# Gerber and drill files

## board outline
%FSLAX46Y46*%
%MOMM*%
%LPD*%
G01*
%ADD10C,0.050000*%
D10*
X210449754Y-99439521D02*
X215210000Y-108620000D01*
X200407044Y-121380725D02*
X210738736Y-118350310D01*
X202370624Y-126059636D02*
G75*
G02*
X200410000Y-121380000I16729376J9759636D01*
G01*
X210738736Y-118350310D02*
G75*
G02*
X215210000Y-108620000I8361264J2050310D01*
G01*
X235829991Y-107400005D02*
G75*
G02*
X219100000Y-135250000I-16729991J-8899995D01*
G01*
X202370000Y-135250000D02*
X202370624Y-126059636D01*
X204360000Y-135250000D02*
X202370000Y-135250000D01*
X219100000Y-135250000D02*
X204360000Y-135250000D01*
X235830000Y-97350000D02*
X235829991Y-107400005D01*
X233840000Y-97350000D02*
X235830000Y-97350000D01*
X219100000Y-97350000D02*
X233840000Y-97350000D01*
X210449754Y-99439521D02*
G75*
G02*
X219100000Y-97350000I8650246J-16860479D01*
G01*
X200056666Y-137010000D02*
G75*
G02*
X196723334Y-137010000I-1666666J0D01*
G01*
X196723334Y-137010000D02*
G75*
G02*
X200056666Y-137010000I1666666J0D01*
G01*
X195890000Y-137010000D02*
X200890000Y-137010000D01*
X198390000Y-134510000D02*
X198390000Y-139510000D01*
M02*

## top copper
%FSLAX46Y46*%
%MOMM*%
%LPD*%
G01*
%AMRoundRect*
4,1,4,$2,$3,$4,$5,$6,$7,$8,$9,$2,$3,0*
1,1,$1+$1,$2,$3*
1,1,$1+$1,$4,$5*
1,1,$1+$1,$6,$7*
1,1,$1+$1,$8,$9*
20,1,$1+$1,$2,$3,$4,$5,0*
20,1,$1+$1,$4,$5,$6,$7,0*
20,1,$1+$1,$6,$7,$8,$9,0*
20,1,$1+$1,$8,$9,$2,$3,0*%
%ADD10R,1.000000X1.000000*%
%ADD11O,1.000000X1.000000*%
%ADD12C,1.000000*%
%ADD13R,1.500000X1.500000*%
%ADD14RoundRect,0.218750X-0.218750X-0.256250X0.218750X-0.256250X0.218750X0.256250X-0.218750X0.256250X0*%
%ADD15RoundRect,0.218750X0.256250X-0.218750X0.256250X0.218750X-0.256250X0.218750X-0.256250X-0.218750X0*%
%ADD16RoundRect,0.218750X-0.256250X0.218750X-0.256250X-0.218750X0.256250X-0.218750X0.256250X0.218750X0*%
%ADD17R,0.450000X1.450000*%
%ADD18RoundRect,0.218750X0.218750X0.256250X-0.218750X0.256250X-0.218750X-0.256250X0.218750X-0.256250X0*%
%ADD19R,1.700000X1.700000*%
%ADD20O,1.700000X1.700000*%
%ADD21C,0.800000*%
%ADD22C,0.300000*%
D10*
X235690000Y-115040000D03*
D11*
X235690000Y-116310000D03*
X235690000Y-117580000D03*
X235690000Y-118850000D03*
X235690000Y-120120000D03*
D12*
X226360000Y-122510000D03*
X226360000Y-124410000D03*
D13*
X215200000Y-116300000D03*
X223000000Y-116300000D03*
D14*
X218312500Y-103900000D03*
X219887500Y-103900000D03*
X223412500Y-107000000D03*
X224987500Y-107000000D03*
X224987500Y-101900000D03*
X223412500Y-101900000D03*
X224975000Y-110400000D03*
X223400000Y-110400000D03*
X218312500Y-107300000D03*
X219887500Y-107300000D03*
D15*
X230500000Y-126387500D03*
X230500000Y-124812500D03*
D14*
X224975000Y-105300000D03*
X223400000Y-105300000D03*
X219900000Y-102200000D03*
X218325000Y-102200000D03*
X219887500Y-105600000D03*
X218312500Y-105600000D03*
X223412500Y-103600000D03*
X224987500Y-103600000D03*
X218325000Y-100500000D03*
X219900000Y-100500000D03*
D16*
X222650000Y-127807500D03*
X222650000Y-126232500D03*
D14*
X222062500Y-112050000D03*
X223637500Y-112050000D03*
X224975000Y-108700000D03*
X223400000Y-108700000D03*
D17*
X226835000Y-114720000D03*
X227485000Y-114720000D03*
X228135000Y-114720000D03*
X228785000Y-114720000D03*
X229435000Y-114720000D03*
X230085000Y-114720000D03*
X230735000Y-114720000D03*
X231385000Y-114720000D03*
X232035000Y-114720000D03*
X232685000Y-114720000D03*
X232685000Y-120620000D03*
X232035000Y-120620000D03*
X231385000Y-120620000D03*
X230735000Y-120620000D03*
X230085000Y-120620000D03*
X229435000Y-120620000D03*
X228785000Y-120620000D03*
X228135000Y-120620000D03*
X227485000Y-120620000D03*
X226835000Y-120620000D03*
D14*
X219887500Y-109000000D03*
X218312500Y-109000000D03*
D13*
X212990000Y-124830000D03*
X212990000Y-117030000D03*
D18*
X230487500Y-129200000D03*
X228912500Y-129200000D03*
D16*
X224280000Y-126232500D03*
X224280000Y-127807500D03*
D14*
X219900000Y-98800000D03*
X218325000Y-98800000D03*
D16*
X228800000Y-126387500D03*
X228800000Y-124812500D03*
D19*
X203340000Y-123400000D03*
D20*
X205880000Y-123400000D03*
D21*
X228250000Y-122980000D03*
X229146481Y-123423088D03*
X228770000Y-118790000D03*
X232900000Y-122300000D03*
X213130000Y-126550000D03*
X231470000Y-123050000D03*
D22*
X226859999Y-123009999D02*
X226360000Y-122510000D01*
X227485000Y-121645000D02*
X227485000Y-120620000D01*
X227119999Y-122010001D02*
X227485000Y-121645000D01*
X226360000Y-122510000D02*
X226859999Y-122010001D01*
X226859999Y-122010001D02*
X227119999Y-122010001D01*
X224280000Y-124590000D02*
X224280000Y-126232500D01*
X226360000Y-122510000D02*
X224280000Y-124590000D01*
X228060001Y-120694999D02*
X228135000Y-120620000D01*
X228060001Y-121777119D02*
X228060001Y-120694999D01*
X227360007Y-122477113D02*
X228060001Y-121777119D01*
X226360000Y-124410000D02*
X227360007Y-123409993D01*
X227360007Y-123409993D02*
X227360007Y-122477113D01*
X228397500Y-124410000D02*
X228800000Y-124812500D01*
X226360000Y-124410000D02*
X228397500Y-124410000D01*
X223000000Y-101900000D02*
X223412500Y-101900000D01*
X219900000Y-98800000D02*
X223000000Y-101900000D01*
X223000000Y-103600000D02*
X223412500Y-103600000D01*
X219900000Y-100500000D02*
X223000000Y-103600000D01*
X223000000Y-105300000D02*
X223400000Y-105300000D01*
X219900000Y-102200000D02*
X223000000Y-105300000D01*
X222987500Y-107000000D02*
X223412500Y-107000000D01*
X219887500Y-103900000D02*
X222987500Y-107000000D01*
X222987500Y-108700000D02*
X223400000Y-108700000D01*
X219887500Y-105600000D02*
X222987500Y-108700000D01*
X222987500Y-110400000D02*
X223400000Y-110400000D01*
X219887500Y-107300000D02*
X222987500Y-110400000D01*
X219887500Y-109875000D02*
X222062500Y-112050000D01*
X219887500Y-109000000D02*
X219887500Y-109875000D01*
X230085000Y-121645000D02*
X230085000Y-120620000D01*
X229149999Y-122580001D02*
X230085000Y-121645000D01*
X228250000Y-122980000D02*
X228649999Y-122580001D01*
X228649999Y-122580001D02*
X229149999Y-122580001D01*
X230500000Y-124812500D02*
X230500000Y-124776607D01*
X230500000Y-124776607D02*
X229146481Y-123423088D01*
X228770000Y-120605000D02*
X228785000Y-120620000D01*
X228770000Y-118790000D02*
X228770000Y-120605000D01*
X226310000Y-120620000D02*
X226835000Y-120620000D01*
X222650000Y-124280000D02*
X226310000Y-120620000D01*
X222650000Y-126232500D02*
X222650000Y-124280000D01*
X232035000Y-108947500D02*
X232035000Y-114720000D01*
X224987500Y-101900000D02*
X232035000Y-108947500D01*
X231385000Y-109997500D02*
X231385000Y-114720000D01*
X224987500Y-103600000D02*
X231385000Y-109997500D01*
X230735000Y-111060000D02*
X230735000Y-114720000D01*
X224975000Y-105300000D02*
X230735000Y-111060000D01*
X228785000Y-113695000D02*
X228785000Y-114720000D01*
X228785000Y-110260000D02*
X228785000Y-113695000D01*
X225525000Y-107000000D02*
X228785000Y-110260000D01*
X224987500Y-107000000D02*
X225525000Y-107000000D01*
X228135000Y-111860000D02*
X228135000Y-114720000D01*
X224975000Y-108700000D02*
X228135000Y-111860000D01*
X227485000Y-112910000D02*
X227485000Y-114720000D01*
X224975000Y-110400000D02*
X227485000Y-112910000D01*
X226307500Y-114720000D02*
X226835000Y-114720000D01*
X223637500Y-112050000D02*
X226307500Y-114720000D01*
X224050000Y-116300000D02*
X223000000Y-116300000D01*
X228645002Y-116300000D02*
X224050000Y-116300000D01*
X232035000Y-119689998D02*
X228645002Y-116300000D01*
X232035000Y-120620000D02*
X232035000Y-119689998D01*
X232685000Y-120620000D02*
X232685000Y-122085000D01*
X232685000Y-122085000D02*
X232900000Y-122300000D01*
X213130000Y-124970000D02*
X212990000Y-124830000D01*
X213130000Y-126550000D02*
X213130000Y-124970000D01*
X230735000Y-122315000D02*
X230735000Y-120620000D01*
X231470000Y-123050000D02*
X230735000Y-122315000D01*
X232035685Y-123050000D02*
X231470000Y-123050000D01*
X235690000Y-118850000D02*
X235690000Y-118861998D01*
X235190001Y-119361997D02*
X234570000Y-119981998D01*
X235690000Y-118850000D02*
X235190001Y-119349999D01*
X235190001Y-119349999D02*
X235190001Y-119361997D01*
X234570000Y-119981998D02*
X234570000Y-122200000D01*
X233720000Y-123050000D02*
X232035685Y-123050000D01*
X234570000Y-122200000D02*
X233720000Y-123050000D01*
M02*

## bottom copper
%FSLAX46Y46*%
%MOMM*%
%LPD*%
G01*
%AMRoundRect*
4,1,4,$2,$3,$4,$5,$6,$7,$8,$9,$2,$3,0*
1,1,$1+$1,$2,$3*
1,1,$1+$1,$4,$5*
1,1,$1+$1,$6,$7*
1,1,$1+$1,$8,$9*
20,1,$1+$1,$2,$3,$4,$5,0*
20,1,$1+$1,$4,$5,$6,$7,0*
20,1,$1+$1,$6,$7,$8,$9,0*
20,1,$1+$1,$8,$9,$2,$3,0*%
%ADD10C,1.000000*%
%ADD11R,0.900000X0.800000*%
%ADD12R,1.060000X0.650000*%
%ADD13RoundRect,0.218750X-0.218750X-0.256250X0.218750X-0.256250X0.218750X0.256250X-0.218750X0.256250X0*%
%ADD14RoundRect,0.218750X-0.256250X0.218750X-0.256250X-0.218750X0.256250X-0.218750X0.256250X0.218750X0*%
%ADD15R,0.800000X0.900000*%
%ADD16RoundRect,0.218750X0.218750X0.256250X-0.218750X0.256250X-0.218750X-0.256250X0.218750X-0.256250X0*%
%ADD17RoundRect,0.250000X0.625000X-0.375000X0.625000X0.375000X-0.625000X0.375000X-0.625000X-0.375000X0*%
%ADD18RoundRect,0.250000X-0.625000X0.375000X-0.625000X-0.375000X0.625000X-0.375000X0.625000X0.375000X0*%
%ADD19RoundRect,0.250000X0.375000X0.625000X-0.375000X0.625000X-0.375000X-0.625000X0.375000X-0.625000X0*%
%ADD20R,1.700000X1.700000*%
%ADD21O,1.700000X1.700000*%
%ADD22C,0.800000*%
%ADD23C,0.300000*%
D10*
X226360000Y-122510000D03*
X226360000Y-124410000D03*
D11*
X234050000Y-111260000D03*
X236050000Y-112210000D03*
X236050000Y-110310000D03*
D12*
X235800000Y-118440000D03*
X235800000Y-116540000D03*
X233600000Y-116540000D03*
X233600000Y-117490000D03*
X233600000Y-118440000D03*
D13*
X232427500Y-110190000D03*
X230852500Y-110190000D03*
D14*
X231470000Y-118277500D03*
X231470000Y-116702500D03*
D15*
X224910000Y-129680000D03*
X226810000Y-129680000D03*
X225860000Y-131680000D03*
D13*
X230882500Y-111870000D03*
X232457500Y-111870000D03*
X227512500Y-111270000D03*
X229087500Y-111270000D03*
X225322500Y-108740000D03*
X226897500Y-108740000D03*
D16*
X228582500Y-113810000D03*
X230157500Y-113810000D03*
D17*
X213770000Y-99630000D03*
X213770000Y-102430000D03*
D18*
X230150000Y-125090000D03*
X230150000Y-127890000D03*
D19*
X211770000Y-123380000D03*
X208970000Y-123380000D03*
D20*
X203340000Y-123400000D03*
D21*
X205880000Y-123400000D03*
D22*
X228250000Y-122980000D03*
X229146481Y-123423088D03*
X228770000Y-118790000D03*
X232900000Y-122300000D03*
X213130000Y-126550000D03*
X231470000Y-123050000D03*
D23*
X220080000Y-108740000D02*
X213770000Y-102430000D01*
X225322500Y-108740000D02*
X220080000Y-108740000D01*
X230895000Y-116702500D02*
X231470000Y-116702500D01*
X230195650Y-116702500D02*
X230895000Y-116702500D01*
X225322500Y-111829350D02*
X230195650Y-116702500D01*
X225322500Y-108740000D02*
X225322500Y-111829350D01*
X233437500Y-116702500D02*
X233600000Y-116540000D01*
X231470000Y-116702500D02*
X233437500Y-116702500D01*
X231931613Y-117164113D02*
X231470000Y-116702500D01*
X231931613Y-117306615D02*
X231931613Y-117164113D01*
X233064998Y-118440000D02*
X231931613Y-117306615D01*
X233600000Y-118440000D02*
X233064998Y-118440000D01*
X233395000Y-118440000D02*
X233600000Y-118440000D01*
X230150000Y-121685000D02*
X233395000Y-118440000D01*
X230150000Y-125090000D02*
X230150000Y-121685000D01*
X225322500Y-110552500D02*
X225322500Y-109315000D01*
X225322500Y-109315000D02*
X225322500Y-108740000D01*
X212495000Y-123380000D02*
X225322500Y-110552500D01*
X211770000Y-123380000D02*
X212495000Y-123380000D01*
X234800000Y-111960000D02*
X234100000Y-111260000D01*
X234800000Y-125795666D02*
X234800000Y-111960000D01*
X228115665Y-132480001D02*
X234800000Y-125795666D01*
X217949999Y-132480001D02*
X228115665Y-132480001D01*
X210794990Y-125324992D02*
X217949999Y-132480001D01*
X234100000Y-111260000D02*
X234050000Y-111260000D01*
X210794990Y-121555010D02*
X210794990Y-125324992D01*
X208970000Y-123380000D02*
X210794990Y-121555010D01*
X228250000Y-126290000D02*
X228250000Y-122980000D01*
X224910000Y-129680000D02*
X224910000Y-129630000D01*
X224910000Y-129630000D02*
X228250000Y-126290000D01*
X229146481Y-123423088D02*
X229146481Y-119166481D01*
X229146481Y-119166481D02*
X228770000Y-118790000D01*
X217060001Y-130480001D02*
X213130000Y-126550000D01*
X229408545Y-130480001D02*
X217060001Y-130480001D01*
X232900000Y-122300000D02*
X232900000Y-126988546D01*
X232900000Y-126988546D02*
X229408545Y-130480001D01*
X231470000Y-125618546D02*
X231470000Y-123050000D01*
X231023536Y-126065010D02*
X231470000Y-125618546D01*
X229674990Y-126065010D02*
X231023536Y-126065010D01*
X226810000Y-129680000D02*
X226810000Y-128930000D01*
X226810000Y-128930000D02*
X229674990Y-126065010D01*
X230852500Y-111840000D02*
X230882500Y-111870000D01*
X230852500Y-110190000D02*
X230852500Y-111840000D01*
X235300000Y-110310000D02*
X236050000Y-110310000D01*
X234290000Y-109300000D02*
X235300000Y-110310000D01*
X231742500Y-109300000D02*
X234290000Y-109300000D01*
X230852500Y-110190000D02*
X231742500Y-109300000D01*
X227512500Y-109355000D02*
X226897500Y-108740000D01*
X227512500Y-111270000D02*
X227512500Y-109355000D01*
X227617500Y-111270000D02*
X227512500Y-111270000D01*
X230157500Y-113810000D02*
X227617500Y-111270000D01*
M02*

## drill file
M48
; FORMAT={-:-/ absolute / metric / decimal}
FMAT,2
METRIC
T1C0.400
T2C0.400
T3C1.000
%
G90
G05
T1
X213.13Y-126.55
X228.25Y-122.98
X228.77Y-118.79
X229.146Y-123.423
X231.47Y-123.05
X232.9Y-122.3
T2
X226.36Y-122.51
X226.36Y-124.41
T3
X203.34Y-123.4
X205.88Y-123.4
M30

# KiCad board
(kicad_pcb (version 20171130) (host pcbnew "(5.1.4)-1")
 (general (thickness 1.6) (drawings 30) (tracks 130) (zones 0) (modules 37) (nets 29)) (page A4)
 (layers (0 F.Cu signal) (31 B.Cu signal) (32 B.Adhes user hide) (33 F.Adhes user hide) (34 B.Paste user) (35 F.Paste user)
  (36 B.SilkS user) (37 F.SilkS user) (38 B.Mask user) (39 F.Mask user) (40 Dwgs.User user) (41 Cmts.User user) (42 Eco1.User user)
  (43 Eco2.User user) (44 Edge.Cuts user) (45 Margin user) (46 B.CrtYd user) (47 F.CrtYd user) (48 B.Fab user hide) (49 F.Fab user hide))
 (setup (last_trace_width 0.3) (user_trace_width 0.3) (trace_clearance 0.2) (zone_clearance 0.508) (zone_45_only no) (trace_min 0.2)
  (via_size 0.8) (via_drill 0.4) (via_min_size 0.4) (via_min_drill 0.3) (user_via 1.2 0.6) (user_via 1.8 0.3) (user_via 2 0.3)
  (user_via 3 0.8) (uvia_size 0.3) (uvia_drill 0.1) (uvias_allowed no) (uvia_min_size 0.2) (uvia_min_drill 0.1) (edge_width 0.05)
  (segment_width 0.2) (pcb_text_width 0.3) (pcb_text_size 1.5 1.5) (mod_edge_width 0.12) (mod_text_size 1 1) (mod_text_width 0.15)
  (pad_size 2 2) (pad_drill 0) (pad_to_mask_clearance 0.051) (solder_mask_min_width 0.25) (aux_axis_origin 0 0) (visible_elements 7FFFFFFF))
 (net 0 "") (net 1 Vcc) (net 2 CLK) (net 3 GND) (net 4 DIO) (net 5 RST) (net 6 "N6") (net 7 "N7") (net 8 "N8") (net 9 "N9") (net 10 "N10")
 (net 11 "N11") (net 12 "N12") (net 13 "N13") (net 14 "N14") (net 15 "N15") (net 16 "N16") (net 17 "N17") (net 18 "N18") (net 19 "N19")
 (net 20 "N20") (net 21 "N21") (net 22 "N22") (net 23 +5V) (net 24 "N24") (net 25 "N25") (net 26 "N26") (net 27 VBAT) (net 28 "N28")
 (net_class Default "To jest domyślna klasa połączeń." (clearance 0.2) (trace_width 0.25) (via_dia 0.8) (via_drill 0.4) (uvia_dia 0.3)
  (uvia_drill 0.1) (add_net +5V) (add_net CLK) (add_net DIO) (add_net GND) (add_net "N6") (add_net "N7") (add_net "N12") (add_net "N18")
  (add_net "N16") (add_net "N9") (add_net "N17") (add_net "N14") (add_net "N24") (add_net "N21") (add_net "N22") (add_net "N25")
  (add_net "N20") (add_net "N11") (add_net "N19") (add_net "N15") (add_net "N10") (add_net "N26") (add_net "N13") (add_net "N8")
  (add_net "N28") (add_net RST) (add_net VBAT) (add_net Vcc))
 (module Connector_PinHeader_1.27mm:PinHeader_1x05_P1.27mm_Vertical (layer F.Cu) (at 235.69 115.04)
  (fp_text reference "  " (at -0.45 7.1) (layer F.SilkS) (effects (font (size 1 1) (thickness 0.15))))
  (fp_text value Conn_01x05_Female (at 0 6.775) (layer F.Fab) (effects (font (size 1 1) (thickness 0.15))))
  (pad 1 smd rect (at 0 0) (size 1 1) (layers F.Cu F.Paste F.Mask) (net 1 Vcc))
  (pad 2 smd oval (at 0 1.27) (size 1 1) (layers F.Cu F.Paste F.Mask) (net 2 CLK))
  (pad 3 smd oval (at 0 2.54) (size 1 1) (layers F.Cu F.Paste F.Mask) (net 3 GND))
  (pad 4 smd oval (at 0 3.81) (size 1 1) (layers F.Cu F.Paste F.Mask) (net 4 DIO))
  (pad 5 smd oval (at 0 5.08) (size 1 1) (layers F.Cu F.Paste F.Mask) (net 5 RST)))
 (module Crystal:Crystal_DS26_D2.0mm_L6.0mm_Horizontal (layer F.Cu) (at 226.36 122.51 270)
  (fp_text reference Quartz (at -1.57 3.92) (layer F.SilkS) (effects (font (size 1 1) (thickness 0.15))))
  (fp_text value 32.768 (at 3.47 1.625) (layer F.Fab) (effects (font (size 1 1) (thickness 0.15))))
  (pad 1 thru_hole circle (at 0 0 270) (size 1 1) (drill 0.4) (layers *.Cu *.Mask) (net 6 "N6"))
  (pad 2 thru_hole circle (at 1.9 0 270) (size 1 1) (drill 0.4) (layers *.Cu *.Mask) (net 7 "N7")))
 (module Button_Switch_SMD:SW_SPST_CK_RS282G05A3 (layer F.Cu) (at 219.1 116.3 180)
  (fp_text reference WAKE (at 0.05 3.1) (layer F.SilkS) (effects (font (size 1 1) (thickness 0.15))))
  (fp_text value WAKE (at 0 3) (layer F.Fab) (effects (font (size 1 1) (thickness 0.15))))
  (pad 2 smd rect (at 3.9 0 180) (size 1.5 1.5) (layers F.Cu F.Paste F.Mask) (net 3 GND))
  (pad 1 smd rect (at -3.9 0 180) (size 1.5 1.5) (layers F.Cu F.Paste F.Mask) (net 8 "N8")))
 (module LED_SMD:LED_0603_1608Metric (layer F.Cu) (at 219.1 103.9)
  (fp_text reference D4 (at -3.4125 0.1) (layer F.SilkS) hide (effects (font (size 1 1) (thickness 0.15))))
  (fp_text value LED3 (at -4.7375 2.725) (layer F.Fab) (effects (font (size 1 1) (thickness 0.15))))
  (pad 1 smd roundrect (at -0.7875 0) (size 0.875 0.95) (layers F.Cu F.Paste F.Mask) (roundrect_rratio 0.25) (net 3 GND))
  (pad 2 smd roundrect (at 0.7875 0) (size 0.875 0.95) (layers F.Cu F.Paste F.Mask) (roundrect_rratio 0.25) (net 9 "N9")))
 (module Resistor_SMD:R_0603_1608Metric (layer F.Cu) (at 224.2 107)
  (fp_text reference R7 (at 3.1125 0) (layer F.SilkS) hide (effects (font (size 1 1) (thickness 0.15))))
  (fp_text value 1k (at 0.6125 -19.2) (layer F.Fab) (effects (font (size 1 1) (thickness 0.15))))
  (pad 1 smd roundrect (at -0.7875 0) (size 0.875 0.95) (layers F.Cu F.Paste F.Mask) (roundrect_rratio 0.25) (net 9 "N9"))
  (pad 2 smd roundrect (at 0.7875 0) (size 0.875 0.95) (layers F.Cu F.Paste F.Mask) (roundrect_rratio 0.25) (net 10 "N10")))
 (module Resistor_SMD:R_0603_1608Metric (layer F.Cu) (at 224.2 101.9)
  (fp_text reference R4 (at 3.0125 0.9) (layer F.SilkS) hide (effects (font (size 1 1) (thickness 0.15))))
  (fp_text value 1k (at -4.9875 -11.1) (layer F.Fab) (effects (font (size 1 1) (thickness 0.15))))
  (pad 2 smd roundrect (at 0.7875 0) (size 0.875 0.95) (layers F.Cu F.Paste F.Mask) (roundrect_rratio 0.25) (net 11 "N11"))
  (pad 1 smd roundrect (at -0.7875 0) (size 0.875 0.95) (layers F.Cu F.Paste F.Mask) (roundrect_rratio 0.25) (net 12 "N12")))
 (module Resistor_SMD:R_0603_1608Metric (layer F.Cu) (at 224.1875 110.4)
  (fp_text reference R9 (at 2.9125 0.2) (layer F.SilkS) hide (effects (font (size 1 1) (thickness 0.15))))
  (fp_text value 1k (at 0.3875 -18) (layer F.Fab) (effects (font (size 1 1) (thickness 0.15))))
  (pad 2 smd roundrect (at 0.7875 0) (size 0.875 0.95) (layers F.Cu F.Paste F.Mask) (roundrect_rratio 0.25) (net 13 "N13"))
  (pad 1 smd roundrect (at -0.7875 0) (size 0.875 0.95) (layers F.Cu F.Paste F.Mask) (roundrect_rratio 0.25) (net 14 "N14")))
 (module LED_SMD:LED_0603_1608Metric (layer F.Cu) (at 219.1 107.3)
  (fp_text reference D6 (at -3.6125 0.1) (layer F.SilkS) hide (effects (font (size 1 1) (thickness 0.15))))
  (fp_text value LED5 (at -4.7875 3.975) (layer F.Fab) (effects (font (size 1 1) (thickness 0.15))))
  (pad 1 smd roundrect (at -0.7875 0) (size 0.875 0.95) (layers F.Cu F.Paste F.Mask) (roundrect_rratio 0.25) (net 3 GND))
  (pad 2 smd roundrect (at 0.7875 0) (size 0.875 0.95) (layers F.Cu F.Paste F.Mask) (roundrect_rratio 0.25) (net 14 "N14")))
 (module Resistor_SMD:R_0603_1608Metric (layer F.Cu) (at 230.5 125.6 90)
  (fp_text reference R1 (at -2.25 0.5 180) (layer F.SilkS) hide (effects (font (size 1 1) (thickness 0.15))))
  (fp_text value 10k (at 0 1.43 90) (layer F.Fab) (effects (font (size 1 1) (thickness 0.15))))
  (pad 1 smd roundrect (at -0.7875 0 90) (size 0.875 0.95) (layers F.Cu F.Paste F.Mask) (roundrect_rratio 0.25) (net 1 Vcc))
  (pad 2 smd roundrect (at 0.7875 0 90) (size 0.875 0.95) (layers F.Cu F.Paste F.Mask) (roundrect_rratio 0.25) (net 5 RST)))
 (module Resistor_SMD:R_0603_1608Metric (layer F.Cu) (at 224.1875 105.3)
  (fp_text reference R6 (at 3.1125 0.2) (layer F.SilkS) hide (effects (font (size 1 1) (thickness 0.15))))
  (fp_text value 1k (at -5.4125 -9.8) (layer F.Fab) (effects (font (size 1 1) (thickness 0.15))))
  (pad 2 smd roundrect (at 0.7875 0) (size 0.875 0.95) (layers F.Cu F.Paste F.Mask) (roundrect_rratio 0.25) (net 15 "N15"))
  (pad 1 smd roundrect (at -0.7875 0) (size 0.875 0.95) (layers F.Cu F.Paste F.Mask) (roundrect_rratio 0.25) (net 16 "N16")))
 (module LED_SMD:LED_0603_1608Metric (layer F.Cu) (at 219.1125 102.2)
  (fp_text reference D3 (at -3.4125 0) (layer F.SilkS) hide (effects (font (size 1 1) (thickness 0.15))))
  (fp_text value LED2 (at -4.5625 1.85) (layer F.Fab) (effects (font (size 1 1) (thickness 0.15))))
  (pad 2 smd roundrect (at 0.7875 0) (size 0.875 0.95) (layers F.Cu F.Paste F.Mask) (roundrect_rratio 0.25) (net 16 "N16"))
  (pad 1 smd roundrect (at -0.7875 0) (size 0.875 0.95) (layers F.Cu F.Paste F.Mask) (roundrect_rratio 0.25) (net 3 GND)))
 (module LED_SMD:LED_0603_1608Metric (layer F.Cu) (at 219.1 105.6)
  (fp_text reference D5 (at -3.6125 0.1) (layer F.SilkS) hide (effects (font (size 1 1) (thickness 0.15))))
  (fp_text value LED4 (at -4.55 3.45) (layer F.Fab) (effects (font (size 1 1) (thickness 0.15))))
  (pad 2 smd roundrect (at 0.7875 0) (size 0.875 0.95) (layers F.Cu F.Paste F.Mask) (roundrect_rratio 0.25) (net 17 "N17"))
  (pad 1 smd roundrect (at -0.7875 0) (size 0.875 0.95) (layers F.Cu F.Paste F.Mask) (roundrect_rratio 0.25) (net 3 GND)))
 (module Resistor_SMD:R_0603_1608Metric (layer F.Cu) (at 224.2 103.6)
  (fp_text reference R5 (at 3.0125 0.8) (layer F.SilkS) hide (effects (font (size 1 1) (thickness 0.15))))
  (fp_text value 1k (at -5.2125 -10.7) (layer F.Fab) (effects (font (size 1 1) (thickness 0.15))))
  (pad 1 smd roundrect (at -0.7875 0) (size 0.875 0.95) (layers F.Cu F.Paste F.Mask) (roundrect_rratio 0.25) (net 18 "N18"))
  (pad 2 smd roundrect (at 0.7875 0) (size 0.875 0.95) (layers F.Cu F.Paste F.Mask) (roundrect_rratio 0.25) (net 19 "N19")))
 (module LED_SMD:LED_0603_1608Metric (layer F.Cu) (at 219.1125 100.5)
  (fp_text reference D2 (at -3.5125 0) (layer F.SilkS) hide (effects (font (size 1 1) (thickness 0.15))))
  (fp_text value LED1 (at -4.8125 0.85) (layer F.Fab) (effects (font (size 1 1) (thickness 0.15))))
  (pad 1 smd roundrect (at -0.7875 0) (size 0.875 0.95) (layers F.Cu F.Paste F.Mask) (roundrect_rratio 0.25) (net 3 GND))
  (pad 2 smd roundrect (at 0.7875 0) (size 0.875 0.95) (layers F.Cu F.Paste F.Mask) (roundrect_rratio 0.25) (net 18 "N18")))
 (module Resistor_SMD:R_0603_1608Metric (layer F.Cu) (at 222.65 127.02 270)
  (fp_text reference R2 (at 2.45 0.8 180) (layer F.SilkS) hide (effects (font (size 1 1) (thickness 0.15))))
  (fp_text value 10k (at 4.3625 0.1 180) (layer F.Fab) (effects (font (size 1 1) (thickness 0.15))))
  (pad 2 smd roundrect (at 0.7875 0 270) (size 0.875 0.95) (layers F.Cu F.Paste F.Mask) (roundrect_rratio 0.25) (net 3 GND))
  (pad 1 smd roundrect (at -0.7875 0 270) (size 0.875 0.95) (layers F.Cu F.Paste F.Mask) (roundrect_rratio 0.25) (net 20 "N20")))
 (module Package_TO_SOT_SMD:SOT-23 (layer B.Cu) (at 235.05 111.26 180)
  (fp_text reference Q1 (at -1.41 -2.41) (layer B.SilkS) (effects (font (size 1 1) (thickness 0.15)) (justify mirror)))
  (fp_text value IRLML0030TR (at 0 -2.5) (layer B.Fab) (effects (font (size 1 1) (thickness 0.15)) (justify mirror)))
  (pad 3 smd rect (at 1 0 180) (size 0.9 0.8) (layers B.Cu B.Paste B.Mask) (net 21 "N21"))
  (pad 2 smd rect (at -1 -0.95 180) (size 0.9 0.8) (layers B.Cu B.Paste B.Mask) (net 3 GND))
  (pad 1 smd rect (at -1 0.95 180) (size 0.9 0.8) (layers B.Cu B.Paste B.Mask) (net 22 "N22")))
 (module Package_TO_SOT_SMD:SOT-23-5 (layer B.Cu) (at 234.7 117.49)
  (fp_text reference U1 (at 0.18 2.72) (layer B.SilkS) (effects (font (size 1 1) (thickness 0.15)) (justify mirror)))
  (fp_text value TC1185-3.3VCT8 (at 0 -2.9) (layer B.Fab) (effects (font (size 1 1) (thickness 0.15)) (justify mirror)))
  (pad 5 smd rect (at 1.1 0.95) (size 1.06 0.65) (layers B.Cu B.Paste B.Mask) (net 1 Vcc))
  (pad 4 smd rect (at 1.1 -0.95) (size 1.06 0.65) (layers B.Cu B.Paste B.Mask))
  (pad 3 smd rect (at -1.1 -0.95) (size 1.06 0.65) (layers B.Cu B.Paste B.Mask) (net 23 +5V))
  (pad 2 smd rect (at -1.1 0) (size 1.06 0.65) (layers B.Cu B.Paste B.Mask) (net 3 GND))
  (pad 1 smd rect (at -1.1 0.95) (size 1.06 0.65) (layers B.Cu B.Paste B.Mask) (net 23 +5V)))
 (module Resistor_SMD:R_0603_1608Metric (layer F.Cu) (at 222.85 112.05)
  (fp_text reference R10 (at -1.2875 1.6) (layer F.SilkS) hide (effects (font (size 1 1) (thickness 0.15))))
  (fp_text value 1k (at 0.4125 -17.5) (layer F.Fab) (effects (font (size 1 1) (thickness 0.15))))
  (pad 1 smd roundrect (at -0.7875 0) (size 0.875 0.95) (layers F.Cu F.Paste F.Mask) (roundrect_rratio 0.25) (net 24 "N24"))
  (pad 2 smd roundrect (at 0.7875 0) (size 0.875 0.95) (layers F.Cu F.Paste F.Mask) (roundrect_rratio 0.25) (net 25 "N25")))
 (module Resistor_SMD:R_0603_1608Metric (layer F.Cu) (at 224.1875 108.7)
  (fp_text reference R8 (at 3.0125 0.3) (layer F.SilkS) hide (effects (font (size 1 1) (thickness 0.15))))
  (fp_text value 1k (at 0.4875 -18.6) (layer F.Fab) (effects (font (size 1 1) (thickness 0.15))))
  (pad 2 smd roundrect (at 0.7875 0) (size 0.875 0.95) (layers F.Cu F.Paste F.Mask) (roundrect_rratio 0.25) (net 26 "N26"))
  (pad 1 smd roundrect (at -0.7875 0) (size 0.875 0.95) (layers F.Cu F.Paste F.Mask) (roundrect_rratio 0.25) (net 17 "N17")))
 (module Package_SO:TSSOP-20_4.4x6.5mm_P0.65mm (layer F.Cu) (at 229.76 117.67 90)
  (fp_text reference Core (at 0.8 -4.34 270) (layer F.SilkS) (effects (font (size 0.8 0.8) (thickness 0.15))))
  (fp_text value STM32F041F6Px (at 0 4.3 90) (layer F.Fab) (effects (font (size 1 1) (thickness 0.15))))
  (pad 20 smd rect (at 2.95 -2.925 90) (size 1.45 0.45) (layers F.Cu F.Paste F.Mask) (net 25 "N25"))
  (pad 19 smd rect (at 2.95 -2.275 90) (size 1.45 0.45) (layers F.Cu F.Paste F.Mask) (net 13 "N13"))
  (pad 18 smd rect (at 2.95 -1.625 90) (size 1.45 0.45) (layers F.Cu F.Paste F.Mask) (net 26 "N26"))
  (pad 17 smd rect (at 2.95 -0.975 90) (size 1.45 0.45) (layers F.Cu F.Paste F.Mask) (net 10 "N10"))
  (pad 16 smd rect (at 2.95 -0.325 90) (size 1.45 0.45) (layers F.Cu F.Paste F.Mask) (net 1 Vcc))
  (pad 15 smd rect (at 2.95 0.325 90) (size 1.45 0.45) (layers F.Cu F.Paste F.Mask) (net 3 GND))
  (pad 14 smd rect (at 2.95 0.975 90) (size 1.45 0.45) (layers F.Cu F.Paste F.Mask) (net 15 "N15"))
  (pad 13 smd rect (at 2.95 1.625 90) (size 1.45 0.45) (layers F.Cu F.Paste F.Mask) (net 19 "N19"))
  (pad 12 smd rect (at 2.95 2.275 90) (size 1.45 0.45) (layers F.Cu F.Paste F.Mask) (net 11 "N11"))
  (pad 11 smd rect (at 2.95 2.925 90) (size 1.45 0.45) (layers F.Cu F.Paste F.Mask) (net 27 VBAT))
  (pad 10 smd rect (at -2.95 2.925 90) (size 1.45 0.45) (layers F.Cu F.Paste F.Mask) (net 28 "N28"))
  (pad 9 smd rect (at -2.95 2.275 90) (size 1.45 0.45) (layers F.Cu F.Paste F.Mask) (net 8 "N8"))
  (pad 8 smd rect (at -2.95 1.625 90) (size 1.45 0.45) (layers F.Cu F.Paste F.Mask))
  (pad 7 smd rect (at -2.95 0.975 90) (size 1.45 0.45) (layers F.Cu F.Paste F.Mask) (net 4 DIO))
  (pad 6 smd rect (at -2.95 0.325 90) (size 1.45 0.45) (layers F.Cu F.Paste F.Mask) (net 2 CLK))
  (pad 5 smd rect (at -2.95 -0.325 90) (size 1.45 0.45) (layers F.Cu F.Paste F.Mask) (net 1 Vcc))
  (pad 4 smd rect (at -2.95 -0.975 90) (size 1.45 0.45) (layers F.Cu F.Paste F.Mask) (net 5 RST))
  (pad 3 smd rect (at -2.95 -1.625 90) (size 1.45 0.45) (layers F.Cu F.Paste F.Mask) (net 7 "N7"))
  (pad 2 smd rect (at -2.95 -2.275 90) (size 1.45 0.45) (layers F.Cu F.Paste F.Mask) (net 6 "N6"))
  (pad 1 smd rect (at -2.95 -2.925 90) (size 1.45 0.45) (layers F.Cu F.Paste F.Mask) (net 20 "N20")))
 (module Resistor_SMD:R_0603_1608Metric (layer B.Cu) (at 231.64 110.19)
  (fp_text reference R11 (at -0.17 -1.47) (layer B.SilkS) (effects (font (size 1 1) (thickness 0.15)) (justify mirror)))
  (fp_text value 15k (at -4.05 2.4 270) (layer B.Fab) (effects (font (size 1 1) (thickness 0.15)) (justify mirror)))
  (pad 2 smd roundrect (at 0.7875 0) (size 0.875 0.95) (layers B.Cu B.Paste B.Mask) (roundrect_rratio 0.25) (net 3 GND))
  (pad 1 smd roundrect (at -0.7875 0) (size 0.875 0.95) (layers B.Cu B.Paste B.Mask) (roundrect_rratio 0.25) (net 22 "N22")))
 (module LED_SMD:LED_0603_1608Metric (layer F.Cu) (at 219.1 109)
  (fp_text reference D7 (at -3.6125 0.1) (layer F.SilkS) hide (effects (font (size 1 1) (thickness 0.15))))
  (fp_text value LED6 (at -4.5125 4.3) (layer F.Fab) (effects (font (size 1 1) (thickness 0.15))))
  (pad 2 smd roundrect (at 0.7875 0) (size 0.875 0.95) (layers F.Cu F.Paste F.Mask) (roundrect_rratio 0.25) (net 24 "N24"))
  (pad 1 smd roundrect (at -0.7875 0) (size 0.875 0.95) (layers F.Cu F.Paste F.Mask) (roundrect_rratio 0.25) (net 3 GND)))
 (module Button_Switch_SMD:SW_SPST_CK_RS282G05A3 (layer F.Cu) (at 212.99 120.93 90)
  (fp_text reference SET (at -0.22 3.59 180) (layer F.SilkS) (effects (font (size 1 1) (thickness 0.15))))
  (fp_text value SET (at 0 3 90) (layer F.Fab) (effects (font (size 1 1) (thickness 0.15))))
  (pad 1 smd rect (at -3.9 0 90) (size 1.5 1.5) (layers F.Cu F.Paste F.Mask) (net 28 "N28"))
  (pad 2 smd rect (at 3.9 0 90) (size 1.5 1.5) (layers F.Cu F.Paste F.Mask) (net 3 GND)))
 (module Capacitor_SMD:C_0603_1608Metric (layer B.Cu) (at 231.47 117.49 270)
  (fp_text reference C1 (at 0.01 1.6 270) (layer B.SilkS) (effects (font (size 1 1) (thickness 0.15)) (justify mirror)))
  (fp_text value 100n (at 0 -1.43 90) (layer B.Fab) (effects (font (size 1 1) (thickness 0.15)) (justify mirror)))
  (pad 2 smd roundrect (at 0.7875 0 270) (size 0.875 0.95) (layers B.Cu B.Paste B.Mask) (roundrect_rratio 0.25) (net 3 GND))
  (pad 1 smd roundrect (at -0.7875 0 270) (size 0.875 0.95) (layers B.Cu B.Paste B.Mask) (roundrect_rratio 0.25) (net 23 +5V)))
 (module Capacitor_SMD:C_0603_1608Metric (layer F.Cu) (at 229.7 129.2 180)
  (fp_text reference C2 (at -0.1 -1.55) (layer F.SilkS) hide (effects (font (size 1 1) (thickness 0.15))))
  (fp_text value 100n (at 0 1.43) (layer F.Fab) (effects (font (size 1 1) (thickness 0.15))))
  (pad 1 smd roundrect (at -0.7875 0 180) (size 0.875 0.95) (layers F.Cu F.Paste F.Mask) (roundrect_rratio 0.25) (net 1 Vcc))
  (pad 2 smd roundrect (at 0.7875 0 180) (size 0.875 0.95) (layers F.Cu F.Paste F.Mask) (roundrect_rratio 0.25) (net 3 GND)))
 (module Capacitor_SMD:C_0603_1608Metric (layer F.Cu) (at 224.28 127.02 270)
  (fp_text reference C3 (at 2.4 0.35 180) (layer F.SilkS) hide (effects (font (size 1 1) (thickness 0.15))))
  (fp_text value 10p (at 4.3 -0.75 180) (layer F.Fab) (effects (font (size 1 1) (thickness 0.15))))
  (pad 1 smd roundrect (at -0.7875 0 270) (size 0.875 0.95) (layers F.Cu F.Paste F.Mask) (roundrect_rratio 0.25) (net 6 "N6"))
  (pad 2 smd roundrect (at 0.7875 0 270) (size 0.875 0.95) (layers F.Cu F.Paste F.Mask) (roundrect_rratio 0.25) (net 3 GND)))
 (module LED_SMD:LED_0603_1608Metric (layer F.Cu) (at 219.1125 98.8)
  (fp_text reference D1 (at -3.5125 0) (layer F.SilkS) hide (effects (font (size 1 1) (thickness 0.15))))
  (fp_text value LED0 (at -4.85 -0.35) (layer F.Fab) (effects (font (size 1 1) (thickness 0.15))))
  (pad 2 smd roundrect (at 0.7875 0) (size 0.875 0.95) (layers F.Cu F.Paste F.Mask) (roundrect_rratio 0.25) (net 12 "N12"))
  (pad 1 smd roundrect (at -0.7875 0) (size 0.875 0.95) (layers F.Cu F.Paste F.Mask) (roundrect_rratio 0.25) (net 3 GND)))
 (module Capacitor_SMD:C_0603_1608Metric (layer F.Cu) (at 228.8 125.6 270)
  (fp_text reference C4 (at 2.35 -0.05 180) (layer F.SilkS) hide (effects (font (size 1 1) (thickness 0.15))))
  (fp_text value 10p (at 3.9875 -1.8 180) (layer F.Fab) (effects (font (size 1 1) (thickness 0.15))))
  (pad 2 smd roundrect (at 0.7875 0 270) (size 0.875 0.95) (layers F.Cu F.Paste F.Mask) (roundrect_rratio 0.25) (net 3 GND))
  (pad 1 smd roundrect (at -0.7875 0 270) (size 0.875 0.95) (layers F.Cu F.Paste F.Mask) (roundrect_rratio 0.25) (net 7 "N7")))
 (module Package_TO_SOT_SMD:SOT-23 (layer B.Cu) (at 225.86 130.68 270)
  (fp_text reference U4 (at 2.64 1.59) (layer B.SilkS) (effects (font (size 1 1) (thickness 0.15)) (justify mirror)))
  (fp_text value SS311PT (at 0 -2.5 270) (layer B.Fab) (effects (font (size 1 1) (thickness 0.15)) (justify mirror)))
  (pad 1 smd rect (at -1 0.95 270) (size 0.9 0.8) (layers B.Cu B.Paste B.Mask) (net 2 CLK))
  (pad 2 smd rect (at -1 -0.95 270) (size 0.9 0.8) (layers B.Cu B.Paste B.Mask) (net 4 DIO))
  (pad 3 smd rect (at 1 0 270) (size 0.9 0.8) (layers B.Cu B.Paste B.Mask) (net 3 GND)))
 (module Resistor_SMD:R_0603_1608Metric (layer B.Cu) (at 231.67 111.87)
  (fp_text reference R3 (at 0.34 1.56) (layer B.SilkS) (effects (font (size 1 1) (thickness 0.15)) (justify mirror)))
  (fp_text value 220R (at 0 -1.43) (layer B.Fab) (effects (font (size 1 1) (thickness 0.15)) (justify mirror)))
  (pad 1 smd roundrect (at -0.7875 0) (size 0.875 0.95) (layers B.Cu B.Paste B.Mask) (roundrect_rratio 0.25) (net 22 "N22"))
  (pad 2 smd roundrect (at 0.7875 0) (size 0.875 0.95) (layers B.Cu B.Paste B.Mask) (roundrect_rratio 0.25) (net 2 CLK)))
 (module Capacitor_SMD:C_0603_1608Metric (layer B.Cu) (at 228.3 111.27)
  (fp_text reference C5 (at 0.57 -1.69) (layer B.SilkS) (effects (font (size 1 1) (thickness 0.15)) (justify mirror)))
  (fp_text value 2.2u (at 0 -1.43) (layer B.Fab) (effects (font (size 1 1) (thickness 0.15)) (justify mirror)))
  (pad 1 smd roundrect (at -0.7875 0) (size 0.875 0.95) (layers B.Cu B.Paste B.Mask) (roundrect_rratio 0.25) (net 27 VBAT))
  (pad 2 smd roundrect (at 0.7875 0) (size 0.875 0.95) (layers B.Cu B.Paste B.Mask) (roundrect_rratio 0.25) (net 3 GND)))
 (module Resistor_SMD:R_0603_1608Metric (layer B.Cu) (at 226.11 108.74)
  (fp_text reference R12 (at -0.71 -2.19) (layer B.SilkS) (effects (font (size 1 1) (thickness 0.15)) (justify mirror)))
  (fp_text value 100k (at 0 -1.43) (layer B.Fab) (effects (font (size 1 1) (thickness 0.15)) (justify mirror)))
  (pad 1 smd roundrect (at -0.7875 0) (size 0.875 0.95) (layers B.Cu B.Paste B.Mask) (roundrect_rratio 0.25) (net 23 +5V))
  (pad 2 smd roundrect (at 0.7875 0) (size 0.875 0.95) (layers B.Cu B.Paste B.Mask) (roundrect_rratio 0.25) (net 27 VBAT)))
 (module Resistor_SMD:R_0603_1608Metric (layer B.Cu) (at 229.37 113.81 180)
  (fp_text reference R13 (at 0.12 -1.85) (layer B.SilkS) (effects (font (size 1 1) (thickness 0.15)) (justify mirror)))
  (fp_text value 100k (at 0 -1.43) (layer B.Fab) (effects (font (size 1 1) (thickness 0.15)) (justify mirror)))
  (pad 2 smd roundrect (at 0.7875 0 180) (size 0.875 0.95) (layers B.Cu B.Paste B.Mask) (roundrect_rratio 0.25) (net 3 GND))
  (pad 1 smd roundrect (at -0.7875 0 180) (size 0.875 0.95) (layers B.Cu B.Paste B.Mask) (roundrect_rratio 0.25) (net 27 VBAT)))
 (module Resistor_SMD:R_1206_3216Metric (layer B.Cu) (at 213.77 101.03 90)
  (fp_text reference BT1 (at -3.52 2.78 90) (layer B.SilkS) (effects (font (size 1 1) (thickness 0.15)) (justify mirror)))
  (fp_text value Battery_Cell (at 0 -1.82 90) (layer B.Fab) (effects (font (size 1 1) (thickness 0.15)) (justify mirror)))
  (pad 2 smd roundrect (at 1.4 0 90) (size 1.25 1.75) (layers B.Cu B.Paste B.Mask) (roundrect_rratio 0.2) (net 3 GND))
  (pad 1 smd roundrect (at -1.4 0 90) (size 1.25 1.75) (layers B.Cu B.Paste B.Mask) (roundrect_rratio 0.2) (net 23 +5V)))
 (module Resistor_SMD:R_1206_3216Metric (layer B.Cu) (at 230.15 126.49 270)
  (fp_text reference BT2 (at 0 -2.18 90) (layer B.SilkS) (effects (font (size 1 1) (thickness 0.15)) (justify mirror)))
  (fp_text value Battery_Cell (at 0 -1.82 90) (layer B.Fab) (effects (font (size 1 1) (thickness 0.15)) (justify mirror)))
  (pad 1 smd roundrect (at -1.4 0 270) (size 1.25 1.75) (layers B.Cu B.Paste B.Mask) (roundrect_rratio 0.2) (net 23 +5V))
  (pad 2 smd roundrect (at 1.4 0 270) (size 1.25 1.75) (layers B.Cu B.Paste B.Mask) (roundrect_rratio 0.2) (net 3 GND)))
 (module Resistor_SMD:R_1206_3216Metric (layer B.Cu) (at 210.37 123.38 180)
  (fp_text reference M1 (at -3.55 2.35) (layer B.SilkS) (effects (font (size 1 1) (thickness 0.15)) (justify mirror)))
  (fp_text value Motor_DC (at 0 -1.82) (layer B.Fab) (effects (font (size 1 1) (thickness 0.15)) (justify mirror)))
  (pad 1 smd roundrect (at -1.4 0 180) (size 1.25 1.75) (layers B.Cu B.Paste B.Mask) (roundrect_rratio 0.2) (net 23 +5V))
  (pad 2 smd roundrect (at 1.4 0 180) (size 1.25 1.75) (layers B.Cu B.Paste B.Mask) (roundrect_rratio 0.2) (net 21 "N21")))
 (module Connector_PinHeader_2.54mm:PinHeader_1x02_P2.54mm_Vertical (layer F.Cu) (at 203.34 123.4 90)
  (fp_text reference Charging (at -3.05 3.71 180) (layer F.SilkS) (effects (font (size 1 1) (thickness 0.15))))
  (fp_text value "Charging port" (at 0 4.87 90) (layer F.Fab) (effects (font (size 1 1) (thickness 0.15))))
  (pad 1 thru_hole rect (at 0 0 90) (size 1.7 1.7) (drill 1) (layers *.Cu *.Mask) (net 3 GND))
  (pad 2 thru_hole oval (at 0 2.54 90) (size 1.7 1.7) (drill 1) (layers *.Cu *.Mask) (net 23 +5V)))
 (gr_line (start 210.449754 99.439521) (end 215.21 108.62) (layer Edge.Cuts) (width 0.05))
 (gr_line (start 200.407044 121.380725) (end 210.738736 118.35031) (layer Edge.Cuts) (width 0.05))
 (gr_arc (start 219.1 116.3) (end 200.41 121.38) (angle -15.05274458) (layer Edge.Cuts) (width 0.05))
 (gr_arc (start 219.1 116.3) (end 215.21 108.62) (angle -76.91524935) (layer Edge.Cuts) (width 0.05))
 (gr_arc (start 219.1 116.3) (end 219.1 135.25) (angle -118.0120165) (layer Edge.Cuts) (width 0.05))
 (gr_line (start 202.37 135.25) (end 202.370624 126.059636) (layer Edge.Cuts) (width 0.05))
 (gr_line (start 204.36 135.25) (end 202.37 135.25) (layer Edge.Cuts) (width 0.05))
 (gr_line (start 219.1 135.25) (end 204.36 135.25) (layer Edge.Cuts) (width 0.05))
 (gr_line (start 235.83 97.35) (end 235.829991 107.400005) (layer Edge.Cuts) (width 0.05))
 (gr_line (start 233.84 97.35) (end 235.83 97.35) (layer Edge.Cuts) (width 0.05))
 (gr_line (start 219.1 97.35) (end 233.84 97.35) (layer Edge.Cuts) (width 0.05))
 (gr_arc (start 219.1 116.3) (end 219.1 97.35) (angle -27.16002962) (layer Edge.Cuts) (width 0.05))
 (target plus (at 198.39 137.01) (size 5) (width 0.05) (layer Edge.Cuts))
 (segment (start 220.08 108.74) (end 213.77 102.43) (width 0.3) (layer B.Cu) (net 23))
 (segment (start 225.3225 108.74) (end 220.08 108.74) (width 0.3) (layer B.Cu) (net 23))
 (segment (start 230.895 116.7025) (end 231.47 116.7025) (width 0.3) (layer B.Cu) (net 23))
 (segment (start 230.19565 116.7025) (end 230.895 116.7025) (width 0.3) (layer B.Cu) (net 23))
 (segment (start 225.3225 111.82935) (end 230.19565 116.7025) (width 0.3) (layer B.Cu) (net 23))
 (segment (start 225.3225 108.74) (end 225.3225 111.82935) (width 0.3) (layer B.Cu) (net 23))
 (segment (start 233.4375 116.7025) (end 233.6 116.54) (width 0.3) (layer B.Cu) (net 23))
 (segment (start 231.47 116.7025) (end 233.4375 116.7025) (width 0.3) (layer B.Cu) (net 23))
 (segment (start 231.931613 117.164113) (end 231.47 116.7025) (width 0.3) (layer B.Cu) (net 23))
 (segment (start 231.931613 117.306615) (end 231.931613 117.164113) (width 0.3) (layer B.Cu) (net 23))
 (segment (start 233.064998 118.44) (end 231.931613 117.306615) (width 0.3) (layer B.Cu) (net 23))
 (segment (start 233.6 118.44) (end 233.064998 118.44) (width 0.3) (layer B.Cu) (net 23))
 (segment (start 233.395 118.44) (end 233.6 118.44) (width 0.3) (layer B.Cu) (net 23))
 (segment (start 230.15 121.685) (end 233.395 118.44) (width 0.3) (layer B.Cu) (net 23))
 (segment (start 230.15 125.09) (end 230.15 121.685) (width 0.3) (layer B.Cu) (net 23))
 (segment (start 225.3225 110.5525) (end 225.3225 109.315) (width 0.3) (layer B.Cu) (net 23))
 (segment (start 225.3225 109.315) (end 225.3225 108.74) (width 0.3) (layer B.Cu) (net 23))
 (segment (start 212.495 123.38) (end 225.3225 110.5525) (width 0.3) (layer B.Cu) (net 23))
 (segment (start 211.77 123.38) (end 212.495 123.38) (width 0.3) (layer B.Cu) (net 23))
 (segment (start 226.859999 123.009999) (end 226.36 122.51) (width 0.3) (layer F.Cu) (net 6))
 (segment (start 227.485 121.645) (end 227.485 120.62) (width 0.3) (layer F.Cu) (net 6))
 (segment (start 227.119999 122.010001) (end 227.485 121.645) (width 0.3) (layer F.Cu) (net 6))
 (segment (start 226.36 122.51) (end 226.859999 122.010001) (width 0.3) (layer F.Cu) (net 6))
 (segment (start 226.859999 122.010001) (end 227.119999 122.010001) (width 0.3) (layer F.Cu) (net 6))
 (segment (start 224.28 124.59) (end 224.28 126.2325) (width 0.3) (layer F.Cu) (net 6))
 (segment (start 226.36 122.51) (end 224.28 124.59) (width 0.3) (layer F.Cu) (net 6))
 (segment (start 228.060001 120.694999) (end 228.135 120.62) (width 0.3) (layer F.Cu) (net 7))
 (segment (start 228.060001 121.777119) (end 228.060001 120.694999) (width 0.3) (layer F.Cu) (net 7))
 (segment (start 227.360007 122.477113) (end 228.060001 121.777119) (width 0.3) (layer F.Cu) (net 7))
 (segment (start 226.36 124.41) (end 227.360007 123.409993) (width 0.3) (layer F.Cu) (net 7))
 (segment (start 227.360007 123.409993) (end 227.360007 122.477113) (width 0.3) (layer F.Cu) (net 7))
 (segment (start 228.3975 124.41) (end 228.8 124.8125) (width 0.3) (layer F.Cu) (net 7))
 (segment (start 226.36 124.41) (end 228.3975 124.41) (width 0.3) (layer F.Cu) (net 7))
 (segment (start 223 101.9) (end 223.4125 101.9) (width 0.3) (layer F.Cu) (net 12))
 (segment (start 219.9 98.8) (end 223 101.9) (width 0.3) (layer F.Cu) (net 12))
 (segment (start 223 103.6) (end 223.4125 103.6) (width 0.3) (layer F.Cu) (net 18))
 (segment (start 219.9 100.5) (end 223 103.6) (width 0.3) (layer F.Cu) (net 18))
 (segment (start 223 105.3) (end 223.4 105.3) (width 0.3) (layer F.Cu) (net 16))
 (segment (start 219.9 102.2) (end 223 105.3) (width 0.3) (layer F.Cu) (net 16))
 (segment (start 222.9875 107) (end 223.4125 107) (width 0.3) (layer F.Cu) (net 9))
 (segment (start 219.8875 103.9) (end 222.9875 107) (width 0.3) (layer F.Cu) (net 9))
 (segment (start 222.9875 108.7) (end 223.4 108.7) (width 0.3) (layer F.Cu) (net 17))
 (segment (start 219.8875 105.6) (end 222.9875 108.7) (width 0.3) (layer F.Cu) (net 17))
 (segment (start 222.9875 110.4) (end 223.4 110.4) (width 0.3) (layer F.Cu) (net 14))
 (segment (start 219.8875 107.3) (end 222.9875 110.4) (width 0.3) (layer F.Cu) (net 14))
 (segment (start 219.8875 109.875) (end 222.0625 112.05) (width 0.3) (layer F.Cu) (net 24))
 (segment (start 219.8875 109) (end 219.8875 109.875) (width 0.3) (layer F.Cu) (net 24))
 (segment (start 234.8 111.96) (end 234.1 111.26) (width 0.3) (layer B.Cu) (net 21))
 (segment (start 234.8 125.795666) (end 234.8 111.96) (width 0.3) (layer B.Cu) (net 21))
 (segment (start 228.115665 132.480001) (end 234.8 125.795666) (width 0.3) (layer B.Cu) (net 21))
 (segment (start 217.949999 132.480001) (end 228.115665 132.480001) (width 0.3) (layer B.Cu) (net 21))
 (segment (start 210.79499 125.324992) (end 217.949999 132.480001) (width 0.3) (layer B.Cu) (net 21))
 (segment (start 234.1 111.26) (end 234.05 111.26) (width 0.3) (layer B.Cu) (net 21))
 (segment (start 210.79499 121.55501) (end 210.79499 125.324992) (width 0.3) (layer B.Cu) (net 21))
 (segment (start 208.97 123.38) (end 210.79499 121.55501) (width 0.3) (layer B.Cu) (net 21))
 (via (at 228.25 122.98) (size 0.8) (drill 0.4) (layers F.Cu B.Cu) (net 2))
 (segment (start 228.25 126.29) (end 228.25 122.98) (width 0.3) (layer B.Cu) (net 2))
 (segment (start 224.91 129.68) (end 224.91 129.63) (width 0.3) (layer B.Cu) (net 2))
 (segment (start 224.91 129.63) (end 228.25 126.29) (width 0.3) (layer B.Cu) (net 2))
 (segment (start 230.085 121.645) (end 230.085 120.62) (width 0.3) (layer F.Cu) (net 2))
 (segment (start 229.149999 122.580001) (end 230.085 121.645) (width 0.3) (layer F.Cu) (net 2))
 (segment (start 228.25 122.98) (end 228.649999 122.580001) (width 0.3) (layer F.Cu) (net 2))
 (segment (start 228.649999 122.580001) (end 229.149999 122.580001) (width 0.3) (layer F.Cu) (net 2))
 (via (at 229.146481 123.423088) (size 0.8) (drill 0.4) (layers F.Cu B.Cu) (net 5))
 (segment (start 230.5 124.8125) (end 230.5 124.776607) (width 0.3) (layer F.Cu) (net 5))
 (segment (start 230.5 124.776607) (end 229.146481 123.423088) (width 0.3) (layer F.Cu) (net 5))
 (via (at 228.77 118.79) (size 0.8) (drill 0.4) (layers F.Cu B.Cu) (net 5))
 (segment (start 229.146481 123.423088) (end 229.146481 119.166481) (width 0.3) (layer B.Cu) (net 5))
 (segment (start 229.146481 119.166481) (end 228.77 118.79) (width 0.3) (layer B.Cu) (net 5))
 (segment (start 228.77 120.605) (end 228.785 120.62) (width 0.3) (layer F.Cu) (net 5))
 (segment (start 228.77 118.79) (end 228.77 120.605) (width 0.3) (layer F.Cu) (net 5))
 (segment (start 226.31 120.62) (end 226.835 120.62) (width 0.3) (layer F.Cu) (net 20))
 (segment (start 222.65 124.28) (end 226.31 120.62) (width 0.3) (layer F.Cu) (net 20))
 (segment (start 222.65 126.2325) (end 222.65 124.28) (width 0.3) (layer F.Cu) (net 20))
 (segment (start 232.035 108.9475) (end 232.035 114.72) (width 0.3) (layer F.Cu) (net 11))
 (segment (start 224.9875 101.9) (end 232.035 108.9475) (width 0.3) (layer F.Cu) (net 11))
 (segment (start 231.385 109.9975) (end 231.385 114.72) (width 0.3) (layer F.Cu) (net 19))
 (segment (start 224.9875 103.6) (end 231.385 109.9975) (width 0.3) (layer F.Cu) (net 19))
 (segment (start 230.735 111.06) (end 230.735 114.72) (width 0.3) (layer F.Cu) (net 15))
 (segment (start 224.975 105.3) (end 230.735 111.06) (width 0.3) (layer F.Cu) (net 15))
 (segment (start 228.785 113.695) (end 228.785 114.72) (width 0.3) (layer F.Cu) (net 10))
 (segment (start 228.785 110.26) (end 228.785 113.695) (width 0.3) (layer F.Cu) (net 10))
 (segment (start 225.525 107) (end 228.785 110.26) (width 0.3) (layer F.Cu) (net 10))
 (segment (start 224.9875 107) (end 225.525 107) (width 0.3) (layer F.Cu) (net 10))
 (segment (start 228.135 111.86) (end 228.135 114.72) (width 0.3) (layer F.Cu) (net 26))
 (segment (start 224.975 108.7) (end 228.135 111.86) (width 0.3) (layer F.Cu) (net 26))
 (segment (start 227.485 112.91) (end 227.485 114.72) (width 0.3) (layer F.Cu) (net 13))
 (segment (start 224.975 110.4) (end 227.485 112.91) (width 0.3) (layer F.Cu) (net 13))
 (segment (start 226.3075 114.72) (end 226.835 114.72) (width 0.3) (layer F.Cu) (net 25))
 (segment (start 223.6375 112.05) (end 226.3075 114.72) (width 0.3) (layer F.Cu) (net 25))
 (segment (start 224.05 116.3) (end 223 116.3) (width 0.3) (layer F.Cu) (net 8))
 (segment (start 228.645002 116.3) (end 224.05 116.3) (width 0.3) (layer F.Cu) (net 8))
 (segment (start 232.035 119.689998) (end 228.645002 116.3) (width 0.3) (layer F.Cu) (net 8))
 (segment (start 232.035 120.62) (end 232.035 119.689998) (width 0.3) (layer F.Cu) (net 8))
 (via (at 232.9 122.3) (size 0.8) (drill 0.4) (layers F.Cu B.Cu) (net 28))
 (segment (start 232.685 120.62) (end 232.685 122.085) (width 0.3) (layer F.Cu) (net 28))
 (segment (start 232.685 122.085) (end 232.9 122.3) (width 0.3) (layer F.Cu) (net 28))
 (via (at 213.13 126.55) (size 0.8) (drill 0.4) (layers F.Cu B.Cu) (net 28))
 (segment (start 217.060001 130.480001) (end 213.13 126.55) (width 0.3) (layer B.Cu) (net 28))
 (segment (start 229.408545 130.480001) (end 217.060001 130.480001) (width 0.3) (layer B.Cu) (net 28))
 (segment (start 232.9 122.3) (end 232.9 126.988546) (width 0.3) (layer B.Cu) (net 28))
 (segment (start 232.9 126.988546) (end 229.408545 130.480001) (width 0.3) (layer B.Cu) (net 28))
 (segment (start 213.13 124.97) (end 212.99 124.83) (width 0.3) (layer F.Cu) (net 28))
 (segment (start 213.13 126.55) (end 213.13 124.97) (width 0.3) (layer F.Cu) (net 28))
 (segment (start 231.47 125.618546) (end 231.47 123.05) (width 0.3) (layer B.Cu) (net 4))
 (via (at 231.47 123.05) (size 0.8) (drill 0.4) (layers F.Cu B.Cu) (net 4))
 (segment (start 231.023536 126.06501) (end 231.47 125.618546) (width 0.3) (layer B.Cu) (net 4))
 (segment (start 229.67499 126.06501) (end 231.023536 126.06501) (width 0.3) (layer B.Cu) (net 4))
 (segment (start 226.81 129.68) (end 226.81 128.93) (width 0.3) (layer B.Cu) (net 4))
 (segment (start 226.81 128.93) (end 229.67499 126.06501) (width 0.3) (layer B.Cu) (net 4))
 (segment (start 230.735 122.315) (end 230.735 120.62) (width 0.3) (layer F.Cu) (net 4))
 (segment (start 231.47 123.05) (end 230.735 122.315) (width 0.3) (layer F.Cu) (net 4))
 (segment (start 232.035685 123.05) (end 231.47 123.05) (width 0.3) (layer F.Cu) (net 4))
 (segment (start 235.69 118.85) (end 235.69 118.861998) (width 0.3) (layer F.Cu) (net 4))
 (segment (start 235.190001 119.361997) (end 234.57 119.981998) (width 0.3) (layer F.Cu) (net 4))
 (segment (start 235.69 118.85) (end 235.190001 119.349999) (width 0.3) (layer F.Cu) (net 4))
 (segment (start 235.190001 119.349999) (end 235.190001 119.361997) (width 0.3) (layer F.Cu) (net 4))
 (segment (start 234.57 119.981998) (end 234.57 122.2) (width 0.3) (layer F.Cu) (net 4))
 (segment (start 233.72 123.05) (end 232.035685 123.05) (width 0.3) (layer F.Cu) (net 4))
 (segment (start 234.57 122.2) (end 233.72 123.05) (width 0.3) (layer F.Cu) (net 4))
 (segment (start 230.8525 111.84) (end 230.8825 111.87) (width 0.3) (layer B.Cu) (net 22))
 (segment (start 230.8525 110.19) (end 230.8525 111.84) (width 0.3) (layer B.Cu) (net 22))
 (segment (start 235.3 110.31) (end 236.05 110.31) (width 0.3) (layer B.Cu) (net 22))
 (segment (start 234.29 109.3) (end 235.3 110.31) (width 0.3) (layer B.Cu) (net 22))
 (segment (start 231.7425 109.3) (end 234.29 109.3) (width 0.3) (layer B.Cu) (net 22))
 (segment (start 230.8525 110.19) (end 231.7425 109.3) (width 0.3) (layer B.Cu) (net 22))
 (segment (start 227.5125 109.355) (end 226.8975 108.74) (width 0.3) (layer B.Cu) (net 27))
 (segment (start 227.5125 111.27) (end 227.5125 109.355) (width 0.3) (layer B.Cu) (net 27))
 (segment (start 227.6175 111.27) (end 227.5125 111.27) (width 0.3) (layer B.Cu) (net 27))
 (segment (start 230.1575 113.81) (end 227.6175 111.27) (width 0.3) (layer B.Cu) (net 27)))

